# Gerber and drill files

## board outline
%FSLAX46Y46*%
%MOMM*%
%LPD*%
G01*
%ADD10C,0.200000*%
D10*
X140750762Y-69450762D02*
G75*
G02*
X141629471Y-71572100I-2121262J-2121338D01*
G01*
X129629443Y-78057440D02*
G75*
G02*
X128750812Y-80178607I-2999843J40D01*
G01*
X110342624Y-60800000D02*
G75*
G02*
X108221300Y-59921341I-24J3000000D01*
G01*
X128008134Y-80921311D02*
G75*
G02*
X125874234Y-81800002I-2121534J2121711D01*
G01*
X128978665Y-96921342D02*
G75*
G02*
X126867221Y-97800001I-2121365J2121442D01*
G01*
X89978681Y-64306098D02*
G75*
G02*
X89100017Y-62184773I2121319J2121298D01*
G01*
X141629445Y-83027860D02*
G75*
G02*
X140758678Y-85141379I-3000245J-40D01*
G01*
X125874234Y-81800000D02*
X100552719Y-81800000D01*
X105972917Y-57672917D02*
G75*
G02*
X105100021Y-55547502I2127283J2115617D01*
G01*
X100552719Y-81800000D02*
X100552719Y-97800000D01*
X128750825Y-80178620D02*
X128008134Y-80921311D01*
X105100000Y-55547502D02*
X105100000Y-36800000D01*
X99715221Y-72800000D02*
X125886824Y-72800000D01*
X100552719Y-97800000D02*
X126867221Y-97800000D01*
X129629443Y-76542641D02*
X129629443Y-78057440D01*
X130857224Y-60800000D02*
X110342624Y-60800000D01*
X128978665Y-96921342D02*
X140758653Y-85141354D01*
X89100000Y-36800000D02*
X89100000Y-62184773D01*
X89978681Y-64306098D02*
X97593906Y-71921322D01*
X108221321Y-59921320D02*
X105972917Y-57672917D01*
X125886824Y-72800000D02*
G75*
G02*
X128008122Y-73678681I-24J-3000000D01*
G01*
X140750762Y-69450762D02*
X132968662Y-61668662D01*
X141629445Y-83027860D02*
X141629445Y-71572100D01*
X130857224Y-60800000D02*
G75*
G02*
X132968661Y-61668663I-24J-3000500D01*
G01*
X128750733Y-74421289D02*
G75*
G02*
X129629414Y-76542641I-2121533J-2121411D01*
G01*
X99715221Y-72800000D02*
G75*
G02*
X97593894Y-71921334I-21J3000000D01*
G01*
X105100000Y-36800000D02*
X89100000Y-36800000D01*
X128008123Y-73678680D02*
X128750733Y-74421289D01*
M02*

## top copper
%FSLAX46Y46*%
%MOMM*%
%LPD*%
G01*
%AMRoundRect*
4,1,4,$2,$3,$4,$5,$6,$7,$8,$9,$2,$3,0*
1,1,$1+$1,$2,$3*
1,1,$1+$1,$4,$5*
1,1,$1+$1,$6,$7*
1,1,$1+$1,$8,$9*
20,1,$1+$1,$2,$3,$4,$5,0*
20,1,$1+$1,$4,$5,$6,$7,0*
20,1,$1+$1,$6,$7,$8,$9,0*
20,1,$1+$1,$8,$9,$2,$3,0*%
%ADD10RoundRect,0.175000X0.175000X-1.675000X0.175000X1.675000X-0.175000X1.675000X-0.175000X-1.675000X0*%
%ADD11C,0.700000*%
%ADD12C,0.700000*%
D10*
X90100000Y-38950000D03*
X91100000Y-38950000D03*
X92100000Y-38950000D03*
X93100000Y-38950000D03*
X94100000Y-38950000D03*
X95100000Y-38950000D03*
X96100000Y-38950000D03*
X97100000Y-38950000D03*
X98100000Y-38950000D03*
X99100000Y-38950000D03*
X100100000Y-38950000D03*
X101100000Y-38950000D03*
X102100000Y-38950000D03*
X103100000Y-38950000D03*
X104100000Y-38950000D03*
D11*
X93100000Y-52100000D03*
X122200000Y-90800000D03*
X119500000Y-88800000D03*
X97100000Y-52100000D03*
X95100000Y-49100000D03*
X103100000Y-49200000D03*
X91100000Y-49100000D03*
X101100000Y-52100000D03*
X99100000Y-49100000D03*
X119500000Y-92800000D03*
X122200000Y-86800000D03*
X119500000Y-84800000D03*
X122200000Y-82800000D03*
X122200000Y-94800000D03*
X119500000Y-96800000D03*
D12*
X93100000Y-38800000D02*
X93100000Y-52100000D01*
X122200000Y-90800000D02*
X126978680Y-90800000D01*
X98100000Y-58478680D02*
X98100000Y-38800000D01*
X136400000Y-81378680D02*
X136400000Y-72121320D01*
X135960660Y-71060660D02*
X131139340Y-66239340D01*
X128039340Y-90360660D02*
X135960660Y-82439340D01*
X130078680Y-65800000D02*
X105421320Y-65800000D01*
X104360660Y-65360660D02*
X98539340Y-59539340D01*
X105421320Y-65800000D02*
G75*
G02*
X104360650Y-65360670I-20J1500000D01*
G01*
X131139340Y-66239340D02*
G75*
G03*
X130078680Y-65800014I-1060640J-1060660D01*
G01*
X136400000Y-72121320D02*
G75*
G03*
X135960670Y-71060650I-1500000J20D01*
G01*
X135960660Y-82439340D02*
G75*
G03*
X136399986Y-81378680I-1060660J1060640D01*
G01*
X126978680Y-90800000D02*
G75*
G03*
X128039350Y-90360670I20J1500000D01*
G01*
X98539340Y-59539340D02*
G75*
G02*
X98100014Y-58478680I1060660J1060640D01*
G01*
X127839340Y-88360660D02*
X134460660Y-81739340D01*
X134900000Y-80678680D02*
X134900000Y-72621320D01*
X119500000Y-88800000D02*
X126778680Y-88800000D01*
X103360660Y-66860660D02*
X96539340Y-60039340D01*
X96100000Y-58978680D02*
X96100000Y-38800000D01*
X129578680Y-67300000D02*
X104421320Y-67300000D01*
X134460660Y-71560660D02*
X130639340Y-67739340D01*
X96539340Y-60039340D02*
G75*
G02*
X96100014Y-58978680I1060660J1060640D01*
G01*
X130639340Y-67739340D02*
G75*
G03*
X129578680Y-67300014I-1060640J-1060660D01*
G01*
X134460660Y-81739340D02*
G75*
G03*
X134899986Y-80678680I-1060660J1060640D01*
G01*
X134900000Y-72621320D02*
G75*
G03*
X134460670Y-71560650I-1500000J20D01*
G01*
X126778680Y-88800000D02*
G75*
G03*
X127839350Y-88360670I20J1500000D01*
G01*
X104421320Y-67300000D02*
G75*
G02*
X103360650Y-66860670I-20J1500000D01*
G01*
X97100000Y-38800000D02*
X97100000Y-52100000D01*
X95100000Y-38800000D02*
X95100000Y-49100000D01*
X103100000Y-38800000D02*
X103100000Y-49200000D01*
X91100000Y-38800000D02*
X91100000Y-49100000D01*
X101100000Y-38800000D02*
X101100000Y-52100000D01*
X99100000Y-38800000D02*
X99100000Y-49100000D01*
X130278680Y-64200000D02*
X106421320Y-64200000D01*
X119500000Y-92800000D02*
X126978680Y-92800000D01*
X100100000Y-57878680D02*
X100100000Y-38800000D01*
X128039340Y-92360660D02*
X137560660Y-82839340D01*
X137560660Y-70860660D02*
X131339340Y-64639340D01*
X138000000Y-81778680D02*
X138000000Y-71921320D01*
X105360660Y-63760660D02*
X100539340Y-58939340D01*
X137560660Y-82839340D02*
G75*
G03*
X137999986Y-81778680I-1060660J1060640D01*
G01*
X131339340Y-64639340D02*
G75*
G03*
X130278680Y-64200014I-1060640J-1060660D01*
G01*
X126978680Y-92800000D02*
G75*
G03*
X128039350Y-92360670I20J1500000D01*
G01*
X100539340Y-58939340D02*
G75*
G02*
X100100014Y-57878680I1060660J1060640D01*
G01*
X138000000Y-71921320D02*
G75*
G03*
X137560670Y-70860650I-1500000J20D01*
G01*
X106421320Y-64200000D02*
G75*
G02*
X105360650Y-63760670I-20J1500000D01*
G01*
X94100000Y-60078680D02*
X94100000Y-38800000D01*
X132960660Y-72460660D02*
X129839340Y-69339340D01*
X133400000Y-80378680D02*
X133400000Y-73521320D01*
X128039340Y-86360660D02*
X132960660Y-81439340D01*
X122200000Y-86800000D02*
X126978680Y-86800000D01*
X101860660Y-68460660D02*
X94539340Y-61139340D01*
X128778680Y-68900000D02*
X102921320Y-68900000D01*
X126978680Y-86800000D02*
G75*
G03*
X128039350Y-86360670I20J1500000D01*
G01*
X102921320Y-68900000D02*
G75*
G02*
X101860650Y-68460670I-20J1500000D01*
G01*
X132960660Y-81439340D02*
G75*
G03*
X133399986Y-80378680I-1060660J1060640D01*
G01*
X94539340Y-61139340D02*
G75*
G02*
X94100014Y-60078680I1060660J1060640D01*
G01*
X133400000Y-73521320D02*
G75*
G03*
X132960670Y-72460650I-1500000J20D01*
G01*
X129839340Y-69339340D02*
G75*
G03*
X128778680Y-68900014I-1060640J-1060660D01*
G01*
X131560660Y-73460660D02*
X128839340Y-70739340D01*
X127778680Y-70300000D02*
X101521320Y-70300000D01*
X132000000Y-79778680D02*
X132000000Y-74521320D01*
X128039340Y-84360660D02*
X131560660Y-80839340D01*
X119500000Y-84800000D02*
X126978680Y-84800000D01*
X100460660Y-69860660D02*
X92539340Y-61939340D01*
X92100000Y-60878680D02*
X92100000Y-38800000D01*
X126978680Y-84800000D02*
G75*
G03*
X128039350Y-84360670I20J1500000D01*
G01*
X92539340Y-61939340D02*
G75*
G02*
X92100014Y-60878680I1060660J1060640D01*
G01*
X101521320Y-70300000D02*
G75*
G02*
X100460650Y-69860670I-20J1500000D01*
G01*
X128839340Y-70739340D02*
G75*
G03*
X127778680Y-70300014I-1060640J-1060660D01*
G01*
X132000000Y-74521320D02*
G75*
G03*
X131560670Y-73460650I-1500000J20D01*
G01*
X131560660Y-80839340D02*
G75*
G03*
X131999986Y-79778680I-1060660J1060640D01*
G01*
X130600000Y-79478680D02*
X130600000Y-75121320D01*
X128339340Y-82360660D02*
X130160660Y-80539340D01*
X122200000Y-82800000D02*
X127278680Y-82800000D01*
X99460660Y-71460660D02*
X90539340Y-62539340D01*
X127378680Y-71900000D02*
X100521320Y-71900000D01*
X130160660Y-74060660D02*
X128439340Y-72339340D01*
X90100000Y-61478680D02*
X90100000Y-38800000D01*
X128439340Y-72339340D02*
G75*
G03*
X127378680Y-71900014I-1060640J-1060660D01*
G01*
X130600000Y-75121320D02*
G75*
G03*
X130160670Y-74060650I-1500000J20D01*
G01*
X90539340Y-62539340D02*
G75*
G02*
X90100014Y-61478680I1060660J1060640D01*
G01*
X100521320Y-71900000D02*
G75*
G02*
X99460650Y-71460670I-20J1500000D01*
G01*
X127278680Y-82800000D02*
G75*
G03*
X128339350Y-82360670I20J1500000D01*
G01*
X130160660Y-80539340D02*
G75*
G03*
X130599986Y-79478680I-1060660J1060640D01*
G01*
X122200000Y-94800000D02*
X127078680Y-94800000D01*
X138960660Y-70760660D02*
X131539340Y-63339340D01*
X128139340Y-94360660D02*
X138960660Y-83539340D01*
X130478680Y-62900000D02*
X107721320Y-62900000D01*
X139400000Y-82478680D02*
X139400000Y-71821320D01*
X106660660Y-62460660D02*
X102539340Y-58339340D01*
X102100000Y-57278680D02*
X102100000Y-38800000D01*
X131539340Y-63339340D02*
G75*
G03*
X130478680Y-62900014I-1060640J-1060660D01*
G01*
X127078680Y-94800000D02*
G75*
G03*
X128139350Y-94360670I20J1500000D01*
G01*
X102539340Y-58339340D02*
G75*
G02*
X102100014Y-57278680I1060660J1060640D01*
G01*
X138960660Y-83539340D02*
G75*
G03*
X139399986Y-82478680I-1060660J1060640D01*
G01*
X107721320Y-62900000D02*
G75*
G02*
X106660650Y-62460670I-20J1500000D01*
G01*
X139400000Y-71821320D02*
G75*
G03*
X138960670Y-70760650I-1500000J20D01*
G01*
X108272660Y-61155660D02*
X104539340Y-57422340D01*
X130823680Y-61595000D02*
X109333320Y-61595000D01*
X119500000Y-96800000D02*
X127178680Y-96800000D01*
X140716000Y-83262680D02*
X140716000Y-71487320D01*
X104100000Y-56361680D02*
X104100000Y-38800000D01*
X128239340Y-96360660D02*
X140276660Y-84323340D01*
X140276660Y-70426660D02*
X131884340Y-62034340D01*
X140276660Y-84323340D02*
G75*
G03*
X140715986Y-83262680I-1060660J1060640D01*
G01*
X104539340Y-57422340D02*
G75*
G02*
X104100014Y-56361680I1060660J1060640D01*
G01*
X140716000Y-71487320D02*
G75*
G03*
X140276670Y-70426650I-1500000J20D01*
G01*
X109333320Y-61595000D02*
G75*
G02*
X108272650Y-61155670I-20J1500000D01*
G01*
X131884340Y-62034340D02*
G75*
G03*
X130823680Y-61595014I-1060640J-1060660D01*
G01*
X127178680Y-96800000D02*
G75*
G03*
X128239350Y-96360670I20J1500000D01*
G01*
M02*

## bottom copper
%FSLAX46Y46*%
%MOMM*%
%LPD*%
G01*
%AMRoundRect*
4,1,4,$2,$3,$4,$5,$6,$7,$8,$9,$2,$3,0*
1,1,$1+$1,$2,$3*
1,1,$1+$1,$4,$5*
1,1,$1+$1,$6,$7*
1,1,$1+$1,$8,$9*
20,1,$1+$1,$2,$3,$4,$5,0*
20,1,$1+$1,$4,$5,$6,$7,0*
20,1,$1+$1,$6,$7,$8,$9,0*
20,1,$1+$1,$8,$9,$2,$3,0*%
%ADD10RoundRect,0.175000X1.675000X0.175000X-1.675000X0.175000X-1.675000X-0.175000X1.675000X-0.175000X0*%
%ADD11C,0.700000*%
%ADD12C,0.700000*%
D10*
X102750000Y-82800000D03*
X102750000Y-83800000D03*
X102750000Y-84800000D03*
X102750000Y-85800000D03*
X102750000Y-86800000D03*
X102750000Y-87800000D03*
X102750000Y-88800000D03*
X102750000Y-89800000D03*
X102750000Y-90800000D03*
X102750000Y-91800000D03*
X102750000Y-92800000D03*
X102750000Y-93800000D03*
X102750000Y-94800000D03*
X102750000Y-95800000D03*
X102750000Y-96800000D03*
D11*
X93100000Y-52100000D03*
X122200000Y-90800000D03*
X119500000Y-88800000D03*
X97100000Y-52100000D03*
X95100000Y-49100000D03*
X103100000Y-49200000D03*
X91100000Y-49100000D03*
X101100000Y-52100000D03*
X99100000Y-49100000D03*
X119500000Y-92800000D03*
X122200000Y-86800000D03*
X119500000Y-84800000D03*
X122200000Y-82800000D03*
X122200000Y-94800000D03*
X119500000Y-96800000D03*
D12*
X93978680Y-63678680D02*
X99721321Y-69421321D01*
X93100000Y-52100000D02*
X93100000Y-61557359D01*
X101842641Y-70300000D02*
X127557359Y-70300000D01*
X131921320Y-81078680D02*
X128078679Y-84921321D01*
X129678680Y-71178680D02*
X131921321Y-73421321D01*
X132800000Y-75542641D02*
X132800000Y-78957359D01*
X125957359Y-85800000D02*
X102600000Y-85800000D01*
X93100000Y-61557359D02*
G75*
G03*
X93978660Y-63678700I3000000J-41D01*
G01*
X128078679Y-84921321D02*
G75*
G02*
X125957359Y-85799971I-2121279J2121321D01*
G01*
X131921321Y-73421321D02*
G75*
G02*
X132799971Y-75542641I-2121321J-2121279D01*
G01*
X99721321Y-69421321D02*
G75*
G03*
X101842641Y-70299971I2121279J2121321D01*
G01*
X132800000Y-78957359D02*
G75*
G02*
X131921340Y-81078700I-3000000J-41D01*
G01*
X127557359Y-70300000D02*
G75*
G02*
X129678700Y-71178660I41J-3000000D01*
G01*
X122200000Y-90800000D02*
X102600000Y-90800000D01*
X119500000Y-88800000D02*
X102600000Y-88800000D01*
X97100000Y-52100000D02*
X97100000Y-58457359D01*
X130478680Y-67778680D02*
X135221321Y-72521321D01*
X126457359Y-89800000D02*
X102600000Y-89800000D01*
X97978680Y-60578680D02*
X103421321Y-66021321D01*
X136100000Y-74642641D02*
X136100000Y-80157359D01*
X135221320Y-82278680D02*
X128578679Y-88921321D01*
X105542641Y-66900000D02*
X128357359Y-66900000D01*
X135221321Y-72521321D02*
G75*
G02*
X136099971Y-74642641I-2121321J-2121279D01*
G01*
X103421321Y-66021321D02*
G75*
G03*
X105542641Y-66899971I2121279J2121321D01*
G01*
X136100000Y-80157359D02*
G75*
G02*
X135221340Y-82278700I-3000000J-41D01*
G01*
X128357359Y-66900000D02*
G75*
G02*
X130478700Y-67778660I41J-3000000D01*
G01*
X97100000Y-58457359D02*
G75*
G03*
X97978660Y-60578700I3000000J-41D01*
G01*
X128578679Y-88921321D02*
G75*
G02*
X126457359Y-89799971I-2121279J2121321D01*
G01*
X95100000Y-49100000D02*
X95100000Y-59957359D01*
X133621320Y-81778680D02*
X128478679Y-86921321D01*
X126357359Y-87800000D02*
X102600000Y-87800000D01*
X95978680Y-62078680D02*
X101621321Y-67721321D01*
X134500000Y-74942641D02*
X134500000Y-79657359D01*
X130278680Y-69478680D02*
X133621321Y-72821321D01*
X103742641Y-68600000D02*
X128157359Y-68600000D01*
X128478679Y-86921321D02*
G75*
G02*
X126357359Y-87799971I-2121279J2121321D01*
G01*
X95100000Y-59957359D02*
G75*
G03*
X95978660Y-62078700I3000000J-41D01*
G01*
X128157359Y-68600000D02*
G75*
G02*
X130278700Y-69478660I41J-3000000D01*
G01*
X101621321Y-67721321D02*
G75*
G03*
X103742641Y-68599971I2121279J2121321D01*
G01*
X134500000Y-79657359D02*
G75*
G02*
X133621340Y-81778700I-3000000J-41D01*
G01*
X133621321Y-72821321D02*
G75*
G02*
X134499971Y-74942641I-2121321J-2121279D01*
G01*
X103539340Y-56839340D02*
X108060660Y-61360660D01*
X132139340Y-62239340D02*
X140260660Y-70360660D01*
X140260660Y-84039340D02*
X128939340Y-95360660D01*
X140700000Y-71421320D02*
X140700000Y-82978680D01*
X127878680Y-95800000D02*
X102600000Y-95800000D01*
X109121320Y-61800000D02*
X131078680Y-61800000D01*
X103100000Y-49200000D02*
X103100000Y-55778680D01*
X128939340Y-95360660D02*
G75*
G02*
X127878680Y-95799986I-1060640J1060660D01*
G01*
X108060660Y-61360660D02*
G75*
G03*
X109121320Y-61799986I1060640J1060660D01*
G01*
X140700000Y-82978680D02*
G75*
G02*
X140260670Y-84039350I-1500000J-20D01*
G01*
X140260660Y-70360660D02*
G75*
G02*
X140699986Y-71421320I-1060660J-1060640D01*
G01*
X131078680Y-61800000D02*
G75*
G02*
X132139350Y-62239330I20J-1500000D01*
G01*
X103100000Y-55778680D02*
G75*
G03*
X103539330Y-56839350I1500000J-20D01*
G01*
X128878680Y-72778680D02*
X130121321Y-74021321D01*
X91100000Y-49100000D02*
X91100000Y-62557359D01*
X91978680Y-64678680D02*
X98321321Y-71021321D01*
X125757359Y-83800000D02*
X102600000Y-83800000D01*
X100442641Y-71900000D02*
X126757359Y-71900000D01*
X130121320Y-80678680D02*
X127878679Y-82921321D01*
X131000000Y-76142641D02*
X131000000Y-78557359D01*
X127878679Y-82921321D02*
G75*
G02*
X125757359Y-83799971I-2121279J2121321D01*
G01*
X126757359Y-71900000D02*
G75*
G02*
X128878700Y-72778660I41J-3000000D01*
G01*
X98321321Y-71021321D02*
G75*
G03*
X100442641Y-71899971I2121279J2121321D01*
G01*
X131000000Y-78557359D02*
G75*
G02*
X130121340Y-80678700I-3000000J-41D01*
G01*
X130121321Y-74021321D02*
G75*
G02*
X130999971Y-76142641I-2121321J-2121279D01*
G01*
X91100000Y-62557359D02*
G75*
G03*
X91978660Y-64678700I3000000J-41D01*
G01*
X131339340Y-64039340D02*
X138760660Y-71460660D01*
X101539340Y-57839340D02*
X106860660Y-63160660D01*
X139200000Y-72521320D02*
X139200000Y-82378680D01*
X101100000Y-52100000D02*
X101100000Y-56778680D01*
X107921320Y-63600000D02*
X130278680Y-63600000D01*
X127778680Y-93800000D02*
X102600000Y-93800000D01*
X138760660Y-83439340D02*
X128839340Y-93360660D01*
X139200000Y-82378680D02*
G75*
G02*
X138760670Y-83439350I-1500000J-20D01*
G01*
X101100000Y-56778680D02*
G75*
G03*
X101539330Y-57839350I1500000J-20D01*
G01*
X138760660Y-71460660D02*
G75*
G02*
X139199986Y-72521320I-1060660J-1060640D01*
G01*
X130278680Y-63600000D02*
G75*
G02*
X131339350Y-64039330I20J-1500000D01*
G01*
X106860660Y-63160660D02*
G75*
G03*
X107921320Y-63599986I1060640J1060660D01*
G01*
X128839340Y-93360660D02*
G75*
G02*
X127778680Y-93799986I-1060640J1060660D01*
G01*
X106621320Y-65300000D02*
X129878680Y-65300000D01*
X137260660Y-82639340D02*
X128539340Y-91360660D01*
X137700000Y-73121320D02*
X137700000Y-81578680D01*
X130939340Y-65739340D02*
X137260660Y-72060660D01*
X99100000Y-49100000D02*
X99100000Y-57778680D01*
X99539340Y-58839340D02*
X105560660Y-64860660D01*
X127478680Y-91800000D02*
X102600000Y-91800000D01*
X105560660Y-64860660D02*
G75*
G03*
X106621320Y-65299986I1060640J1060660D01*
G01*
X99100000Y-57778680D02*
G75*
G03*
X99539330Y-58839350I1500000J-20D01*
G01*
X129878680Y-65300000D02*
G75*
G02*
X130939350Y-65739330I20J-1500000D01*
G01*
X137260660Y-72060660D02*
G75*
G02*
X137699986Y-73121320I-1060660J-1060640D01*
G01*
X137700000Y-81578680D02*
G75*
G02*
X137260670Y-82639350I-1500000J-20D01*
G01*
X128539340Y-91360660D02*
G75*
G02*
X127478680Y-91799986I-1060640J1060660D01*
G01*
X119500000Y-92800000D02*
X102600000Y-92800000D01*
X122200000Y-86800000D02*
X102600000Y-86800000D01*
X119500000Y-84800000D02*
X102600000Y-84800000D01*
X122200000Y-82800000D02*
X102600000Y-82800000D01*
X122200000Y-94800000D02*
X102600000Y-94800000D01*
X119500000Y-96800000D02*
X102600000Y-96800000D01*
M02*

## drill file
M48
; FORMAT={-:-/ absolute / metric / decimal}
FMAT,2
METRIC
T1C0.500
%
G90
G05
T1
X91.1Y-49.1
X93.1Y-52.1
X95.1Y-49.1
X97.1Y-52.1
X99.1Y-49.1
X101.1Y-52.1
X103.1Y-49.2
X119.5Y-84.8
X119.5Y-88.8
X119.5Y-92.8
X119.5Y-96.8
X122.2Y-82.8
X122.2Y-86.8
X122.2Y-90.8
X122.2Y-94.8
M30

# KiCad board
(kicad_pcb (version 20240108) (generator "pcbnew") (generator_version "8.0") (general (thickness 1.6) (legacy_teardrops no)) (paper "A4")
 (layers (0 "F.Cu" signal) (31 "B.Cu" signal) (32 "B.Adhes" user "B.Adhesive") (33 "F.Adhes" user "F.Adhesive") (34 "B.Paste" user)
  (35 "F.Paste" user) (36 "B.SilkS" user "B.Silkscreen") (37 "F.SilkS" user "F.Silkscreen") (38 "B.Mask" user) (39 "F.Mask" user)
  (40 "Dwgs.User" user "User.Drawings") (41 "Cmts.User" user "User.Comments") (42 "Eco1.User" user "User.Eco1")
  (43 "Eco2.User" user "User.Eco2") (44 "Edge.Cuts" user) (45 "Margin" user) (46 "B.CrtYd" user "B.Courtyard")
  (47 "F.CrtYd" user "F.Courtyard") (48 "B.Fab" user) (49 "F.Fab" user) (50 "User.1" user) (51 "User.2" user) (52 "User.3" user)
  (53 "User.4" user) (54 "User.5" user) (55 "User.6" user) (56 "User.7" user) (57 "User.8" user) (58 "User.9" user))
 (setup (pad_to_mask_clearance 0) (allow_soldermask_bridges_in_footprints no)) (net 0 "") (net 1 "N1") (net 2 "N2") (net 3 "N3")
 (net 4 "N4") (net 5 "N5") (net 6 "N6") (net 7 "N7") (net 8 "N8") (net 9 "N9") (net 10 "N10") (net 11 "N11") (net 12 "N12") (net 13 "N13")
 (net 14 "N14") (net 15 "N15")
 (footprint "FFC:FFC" (layer "F.Cu") (at 97.1 38.8 90)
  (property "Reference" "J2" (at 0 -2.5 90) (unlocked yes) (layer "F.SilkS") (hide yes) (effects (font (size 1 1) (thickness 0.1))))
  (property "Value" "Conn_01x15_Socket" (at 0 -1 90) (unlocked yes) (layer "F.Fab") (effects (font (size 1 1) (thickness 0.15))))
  (pad "1" smd roundrect (at -0.15 -7 90) (size 3.7 0.7) (layers "F.Cu" "F.Paste" "F.Mask") (roundrect_rratio 0.25) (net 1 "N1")
   (thermal_bridge_angle 45))
  (pad "2" smd roundrect (at -0.15 -6 90) (size 3.7 0.7) (layers "F.Cu" "F.Paste" "F.Mask") (roundrect_rratio 0.25) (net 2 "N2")
   (thermal_bridge_angle 45))
  (pad "3" smd roundrect (at -0.15 -5 90) (size 3.7 0.7) (layers "F.Cu" "F.Paste" "F.Mask") (roundrect_rratio 0.25) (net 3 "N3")
   (thermal_bridge_angle 45))
  (pad "4" smd roundrect (at -0.15 -4 90) (size 3.7 0.7) (layers "F.Cu" "F.Paste" "F.Mask") (roundrect_rratio 0.25) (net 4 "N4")
   (thermal_bridge_angle 45))
  (pad "5" smd roundrect (at -0.15 -3 90) (size 3.7 0.7) (layers "F.Cu" "F.Paste" "F.Mask") (roundrect_rratio 0.25) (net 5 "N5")
   (thermal_bridge_angle 45))
  (pad "6" smd roundrect (at -0.15 -2 90) (size 3.7 0.7) (layers "F.Cu" "F.Paste" "F.Mask") (roundrect_rratio 0.25) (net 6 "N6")
   (thermal_bridge_angle 45))
  (pad "7" smd roundrect (at -0.15 -1 90) (size 3.7 0.7) (layers "F.Cu" "F.Paste" "F.Mask") (roundrect_rratio 0.25) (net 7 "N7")
   (thermal_bridge_angle 45))
  (pad "8" smd roundrect (at -0.15 0 90) (size 3.7 0.7) (layers "F.Cu" "F.Paste" "F.Mask") (roundrect_rratio 0.25) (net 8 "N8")
   (thermal_bridge_angle 45))
  (pad "9" smd roundrect (at -0.15 1 90) (size 3.7 0.7) (layers "F.Cu" "F.Paste" "F.Mask") (roundrect_rratio 0.25) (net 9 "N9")
   (thermal_bridge_angle 45))
  (pad "10" smd roundrect (at -0.15 2 90) (size 3.7 0.7) (layers "F.Cu" "F.Paste" "F.Mask") (roundrect_rratio 0.25) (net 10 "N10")
   (thermal_bridge_angle 45))
  (pad "11" smd roundrect (at -0.15 3 90) (size 3.7 0.7) (layers "F.Cu" "F.Paste" "F.Mask") (roundrect_rratio 0.25) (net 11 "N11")
   (thermal_bridge_angle 45))
  (pad "12" smd roundrect (at -0.15 4 90) (size 3.7 0.7) (layers "F.Cu" "F.Paste" "F.Mask") (roundrect_rratio 0.25) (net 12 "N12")
   (thermal_bridge_angle 45))
  (pad "13" smd roundrect (at -0.15 5 90) (size 3.7 0.7) (layers "F.Cu" "F.Paste" "F.Mask") (roundrect_rratio 0.25) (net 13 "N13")
   (thermal_bridge_angle 45))
  (pad "14" smd roundrect (at -0.15 6 90) (size 3.7 0.7) (layers "F.Cu" "F.Paste" "F.Mask") (roundrect_rratio 0.25) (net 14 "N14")
   (thermal_bridge_angle 45))
  (pad "15" smd roundrect (at -0.15 7 90) (size 3.7 0.7) (layers "F.Cu" "F.Paste" "F.Mask") (roundrect_rratio 0.25) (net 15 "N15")
   (thermal_bridge_angle 45)))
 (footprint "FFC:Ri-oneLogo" (layer "F.Cu") (at 111.1 69.2)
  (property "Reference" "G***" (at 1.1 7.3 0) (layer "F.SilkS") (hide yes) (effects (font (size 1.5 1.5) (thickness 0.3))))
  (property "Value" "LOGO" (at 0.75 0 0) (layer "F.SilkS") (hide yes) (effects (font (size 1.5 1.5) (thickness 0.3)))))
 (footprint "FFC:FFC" (layer "B.Cu") (at 102.6 89.8 180)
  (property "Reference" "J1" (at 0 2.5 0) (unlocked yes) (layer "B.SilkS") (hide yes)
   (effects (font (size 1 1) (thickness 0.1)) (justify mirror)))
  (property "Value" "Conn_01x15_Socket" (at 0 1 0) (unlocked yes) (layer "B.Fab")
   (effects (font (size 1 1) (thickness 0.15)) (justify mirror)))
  (pad "1" smd roundrect (at -0.15 7 180) (size 3.7 0.7) (layers "B.Cu" "B.Paste" "B.Mask") (roundrect_rratio 0.25) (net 1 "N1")
   (thermal_bridge_angle 45))
  (pad "2" smd roundrect (at -0.15 6 180) (size 3.7 0.7) (layers "B.Cu" "B.Paste" "B.Mask") (roundrect_rratio 0.25) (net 2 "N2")
   (thermal_bridge_angle 45))
  (pad "3" smd roundrect (at -0.15 5 180) (size 3.7 0.7) (layers "B.Cu" "B.Paste" "B.Mask") (roundrect_rratio 0.25) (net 3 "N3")
   (thermal_bridge_angle 45))
  (pad "4" smd roundrect (at -0.15 4 180) (size 3.7 0.7) (layers "B.Cu" "B.Paste" "B.Mask") (roundrect_rratio 0.25) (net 4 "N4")
   (thermal_bridge_angle 45))
  (pad "5" smd roundrect (at -0.15 3 180) (size 3.7 0.7) (layers "B.Cu" "B.Paste" "B.Mask") (roundrect_rratio 0.25) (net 5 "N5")
   (thermal_bridge_angle 45))
  (pad "6" smd roundrect (at -0.15 2 180) (size 3.7 0.7) (layers "B.Cu" "B.Paste" "B.Mask") (roundrect_rratio 0.25) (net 6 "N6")
   (thermal_bridge_angle 45))
  (pad "7" smd roundrect (at -0.15 1 180) (size 3.7 0.7) (layers "B.Cu" "B.Paste" "B.Mask") (roundrect_rratio 0.25) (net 7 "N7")
   (thermal_bridge_angle 45))
  (pad "8" smd roundrect (at -0.15 0 180) (size 3.7 0.7) (layers "B.Cu" "B.Paste" "B.Mask") (roundrect_rratio 0.25) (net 8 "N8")
   (thermal_bridge_angle 45))
  (pad "9" smd roundrect (at -0.15 -1 180) (size 3.7 0.7) (layers "B.Cu" "B.Paste" "B.Mask") (roundrect_rratio 0.25) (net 9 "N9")
   (thermal_bridge_angle 45))
  (pad "10" smd roundrect (at -0.15 -2 180) (size 3.7 0.7) (layers "B.Cu" "B.Paste" "B.Mask") (roundrect_rratio 0.25) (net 10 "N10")
   (thermal_bridge_angle 45))
  (pad "11" smd roundrect (at -0.15 -3 180) (size 3.7 0.7) (layers "B.Cu" "B.Paste" "B.Mask") (roundrect_rratio 0.25) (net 11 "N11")
   (thermal_bridge_angle 45))
  (pad "12" smd roundrect (at -0.15 -4 180) (size 3.7 0.7) (layers "B.Cu" "B.Paste" "B.Mask") (roundrect_rratio 0.25) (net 12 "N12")
   (thermal_bridge_angle 45))
  (pad "13" smd roundrect (at -0.15 -5 180) (size 3.7 0.7) (layers "B.Cu" "B.Paste" "B.Mask") (roundrect_rratio 0.25) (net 13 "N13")
   (thermal_bridge_angle 45))
  (pad "14" smd roundrect (at -0.15 -6 180) (size 3.7 0.7) (layers "B.Cu" "B.Paste" "B.Mask") (roundrect_rratio 0.25) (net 14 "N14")
   (thermal_bridge_angle 45))
  (pad "15" smd roundrect (at -0.15 -7 180) (size 3.7 0.7) (layers "B.Cu" "B.Paste" "B.Mask") (roundrect_rratio 0.25) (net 15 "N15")
   (thermal_bridge_angle 45)))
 (gr_arc (start 140.750762 69.450762) (mid 141.401086 70.42404) (end 141.629445 71.5721) (stroke (width 0.2) (type default))
  (layer "Edge.Cuts"))
 (gr_arc (start 129.629443 78.05744) (mid 129.401097 79.205413) (end 128.750825 80.17862) (stroke (width 0.2) (type default))
  (layer "Edge.Cuts"))
 (gr_arc (start 110.342624 60.8) (mid 109.194585 60.571635) (end 108.221321 59.92132) (stroke (width 0.2) (type default))
  (layer "Edge.Cuts"))
 (gr_arc (start 128.008134 80.921311) (mid 127.029045 81.574019) (end 125.874234 81.8) (stroke (width 0.2) (type default))
  (layer "Edge.Cuts"))
 (gr_arc (start 128.978665 96.921342) (mid 128.009955 97.569757) (end 126.867221 97.8) (stroke (width 0.2) (type default))
  (layer "Edge.Cuts"))
 (gr_arc (start 89.978681 64.306098) (mid 89.328361 63.332826) (end 89.1 62.184773) (stroke (width 0.2) (type default)) (layer "Edge.Cuts"))
 (gr_arc (start 141.629445 83.02786) (mid 141.403217 84.170787) (end 140.758653 85.141354) (stroke (width 0.2) (type default))
  (layer "Edge.Cuts"))
 (gr_line (start 125.874234 81.8) (end 100.552719 81.8) (stroke (width 0.2) (type default)) (layer "Edge.Cuts"))
 (gr_arc (start 105.972917 57.672917) (mid 105.324931 56.697085) (end 105.1 55.547502) (stroke (width 0.2) (type default))
  (layer "Edge.Cuts"))
 (gr_line (start 100.552719 81.8) (end 100.552719 97.8) (stroke (width 0.2) (type default)) (layer "Edge.Cuts"))
 (gr_line (start 128.750825 80.17862) (end 128.008134 80.921311) (stroke (width 0.2) (type default)) (layer "Edge.Cuts"))
 (gr_line (start 105.1 55.547502) (end 105.1 36.8) (stroke (width 0.2) (type default)) (layer "Edge.Cuts"))
 (gr_line (start 99.715221 72.8) (end 125.886824 72.8) (stroke (width 0.2) (type default)) (layer "Edge.Cuts"))
 (gr_line (start 100.552719 97.8) (end 126.867221 97.8) (stroke (width 0.2) (type default)) (layer "Edge.Cuts"))
 (gr_line (start 129.629443 76.542641) (end 129.629443 78.05744) (stroke (width 0.2) (type default)) (layer "Edge.Cuts"))
 (gr_line (start 130.857224 60.8) (end 110.342624 60.8) (stroke (width 0.2) (type default)) (layer "Edge.Cuts"))
 (gr_line (start 128.978665 96.921342) (end 140.758653 85.141354) (stroke (width 0.2) (type default)) (layer "Edge.Cuts"))
 (gr_line (start 89.1 36.8) (end 89.1 62.184773) (stroke (width 0.2) (type default)) (layer "Edge.Cuts"))
 (gr_line (start 89.978681 64.306098) (end 97.593906 71.921322) (stroke (width 0.2) (type default)) (layer "Edge.Cuts"))
 (gr_line (start 108.221321 59.92132) (end 105.972917 57.672917) (stroke (width 0.2) (type default)) (layer "Edge.Cuts"))
 (gr_arc (start 125.886824 72.8) (mid 127.034862 73.028364) (end 128.008123 73.67868) (stroke (width 0.2) (type default))
  (layer "Edge.Cuts"))
 (gr_line (start 140.750762 69.450762) (end 132.968662 61.668662) (stroke (width 0.2) (type default)) (layer "Edge.Cuts"))
 (gr_line (start 141.629445 83.02786) (end 141.629445 71.5721) (stroke (width 0.2) (type default)) (layer "Edge.Cuts"))
 (gr_arc (start 130.857224 60.8) (mid 131.998793 61.025653) (end 132.968662 61.668662) (stroke (width 0.2) (type default))
  (layer "Edge.Cuts"))
 (gr_arc (start 128.750733 74.421289) (mid 129.401057 75.394574) (end 129.629443 76.542641) (stroke (width 0.2) (type default))
  (layer "Edge.Cuts"))
 (gr_arc (start 99.715221 72.8) (mid 98.567174 72.571639) (end 97.593906 71.921322) (stroke (width 0.2) (type default)) (layer "Edge.Cuts"))
 (gr_line (start 105.1 36.8) (end 89.1 36.8) (stroke (width 0.2) (type default)) (layer "Edge.Cuts"))
 (gr_line (start 128.008123 73.67868) (end 128.750733 74.421289) (stroke (width 0.2) (type default)) (layer "Edge.Cuts"))
 (segment (start 93.1 38.8) (end 93.1 52.1) (width 0.7) (layer "F.Cu") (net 4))
 (via (at 93.1 52.1) (size 0.7) (drill 0.5) (layers "F.Cu" "B.Cu") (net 4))
 (segment (start 93.97868 63.67868) (end 99.721321 69.421321) (width 0.7) (layer "B.Cu") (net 4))
 (segment (start 93.1 52.1) (end 93.1 61.557359) (width 0.7) (layer "B.Cu") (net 4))
 (segment (start 101.842641 70.3) (end 127.557359 70.3) (width 0.7) (layer "B.Cu") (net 4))
 (segment (start 131.92132 81.07868) (end 128.078679 84.921321) (width 0.7) (layer "B.Cu") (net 4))
 (segment (start 129.67868 71.17868) (end 131.921321 73.421321) (width 0.7) (layer "B.Cu") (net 4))
 (segment (start 132.8 75.542641) (end 132.8 78.957359) (width 0.7) (layer "B.Cu") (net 4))
 (segment (start 125.957359 85.8) (end 102.6 85.8) (width 0.7) (layer "B.Cu") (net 4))
 (arc (start 93.1 61.557359) (mid 93.328362 62.70541) (end 93.97868 63.67868) (width 0.7) (layer "B.Cu") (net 4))
 (arc (start 128.078679 84.921321) (mid 127.105409 85.571639) (end 125.957359 85.8) (width 0.7) (layer "B.Cu") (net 4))
 (arc (start 131.921321 73.421321) (mid 132.571639 74.394591) (end 132.8 75.542641) (width 0.7) (layer "B.Cu") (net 4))
 (arc (start 99.721321 69.421321) (mid 100.694591 70.071639) (end 101.842641 70.3) (width 0.7) (layer "B.Cu") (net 4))
 (arc (start 132.8 78.957359) (mid 132.571638 80.10541) (end 131.92132 81.07868) (width 0.7) (layer "B.Cu") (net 4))
 (arc (start 127.557359 70.3) (mid 128.70541 70.528362) (end 129.67868 71.17868) (width 0.7) (layer "B.Cu") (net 4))
 (segment (start 122.2 90.8) (end 126.97868 90.8) (width 0.7) (layer "F.Cu") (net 9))
 (segment (start 98.1 58.47868) (end 98.1 38.8) (width 0.7) (layer "F.Cu") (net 9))
 (segment (start 136.4 81.37868) (end 136.4 72.12132) (width 0.7) (layer "F.Cu") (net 9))
 (segment (start 135.96066 71.06066) (end 131.13934 66.23934) (width 0.7) (layer "F.Cu") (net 9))
 (segment (start 128.03934 90.36066) (end 135.96066 82.43934) (width 0.7) (layer "F.Cu") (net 9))
 (segment (start 130.07868 65.8) (end 105.42132 65.8) (width 0.7) (layer "F.Cu") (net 9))
 (segment (start 104.36066 65.36066) (end 98.53934 59.53934) (width 0.7) (layer "F.Cu") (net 9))
 (via (at 122.2 90.8) (size 0.7) (drill 0.5) (layers "F.Cu" "B.Cu") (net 9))
 (arc (start 105.42132 65.8) (mid 104.847295 65.685819) (end 104.36066 65.36066) (width 0.7) (layer "F.Cu") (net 9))
 (arc (start 131.13934 66.23934) (mid 130.652705 65.914181) (end 130.07868 65.8) (width 0.7) (layer "F.Cu") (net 9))
 (arc (start 136.4 72.12132) (mid 136.285819 71.547295) (end 135.96066 71.06066) (width 0.7) (layer "F.Cu") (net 9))
 (arc (start 135.96066 82.43934) (mid 136.285819 81.952705) (end 136.4 81.37868) (width 0.7) (layer "F.Cu") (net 9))
 (arc (start 126.97868 90.8) (mid 127.552705 90.685819) (end 128.03934 90.36066) (width 0.7) (layer "F.Cu") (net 9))
 (arc (start 98.53934 59.53934) (mid 98.214181 59.052705) (end 98.1 58.47868) (width 0.7) (layer "F.Cu") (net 9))
 (segment (start 122.2 90.8) (end 102.6 90.8) (width 0.7) (layer "B.Cu") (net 9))
 (segment (start 127.83934 88.36066) (end 134.46066 81.73934) (width 0.7) (layer "F.Cu") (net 7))
 (segment (start 134.9 80.67868) (end 134.9 72.62132) (width 0.7) (layer "F.Cu") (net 7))
 (segment (start 119.5 88.8) (end 126.77868 88.8) (width 0.7) (layer "F.Cu") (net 7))
 (segment (start 103.36066 66.86066) (end 96.53934 60.03934) (width 0.7) (layer "F.Cu") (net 7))
 (segment (start 96.1 58.97868) (end 96.1 38.8) (width 0.7) (layer "F.Cu") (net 7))
 (segment (start 129.57868 67.3) (end 104.42132 67.3) (width 0.7) (layer "F.Cu") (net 7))
 (segment (start 134.46066 71.56066) (end 130.63934 67.73934) (width 0.7) (layer "F.Cu") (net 7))
 (via (at 119.5 88.8) (size 0.7) (drill 0.5) (layers "F.Cu" "B.Cu") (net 7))
 (arc (start 96.53934 60.03934) (mid 96.214181 59.552705) (end 96.1 58.97868) (width 0.7) (layer "F.Cu") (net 7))
 (arc (start 130.63934 67.73934) (mid 130.152705 67.414181) (end 129.57868 67.3) (width 0.7) (layer "F.Cu") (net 7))
 (arc (start 134.46066 81.73934) (mid 134.785819 81.252705) (end 134.9 80.67868) (width 0.7) (layer "F.Cu") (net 7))
 (arc (start 134.9 72.62132) (mid 134.785819 72.047295) (end 134.46066 71.56066) (width 0.7) (layer "F.Cu") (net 7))
 (arc (start 126.77868 88.8) (mid 127.352705 88.685819) (end 127.83934 88.36066) (width 0.7) (layer "F.Cu") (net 7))
 (arc (start 104.42132 67.3) (mid 103.847295 67.185819) (end 103.36066 66.86066) (width 0.7) (layer "F.Cu") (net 7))
 (segment (start 119.5 88.8) (end 102.6 88.8) (width 0.7) (layer "B.Cu") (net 7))
 (segment (start 97.1 38.8) (end 97.1 52.1) (width 0.7) (layer "F.Cu") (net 8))
 (via (at 97.1 52.1) (size 0.7) (drill 0.5) (layers "F.Cu" "B.Cu") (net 8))
 (segment (start 97.1 52.1) (end 97.1 58.457359) (width 0.7) (layer "B.Cu") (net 8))
 (segment (start 130.47868 67.77868) (end 135.221321 72.521321) (width 0.7) (layer "B.Cu") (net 8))
 (segment (start 126.457359 89.8) (end 102.6 89.8) (width 0.7) (layer "B.Cu") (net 8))
 (segment (start 97.97868 60.57868) (end 103.421321 66.021321) (width 0.7) (layer "B.Cu") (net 8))
 (segment (start 136.1 74.642641) (end 136.1 80.157359) (width 0.7) (layer "B.Cu") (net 8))
 (segment (start 135.22132 82.27868) (end 128.578679 88.921321) (width 0.7) (layer "B.Cu") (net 8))
 (segment (start 105.542641 66.9) (end 128.357359 66.9) (width 0.7) (layer "B.Cu") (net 8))
 (arc (start 135.221321 72.521321) (mid 135.871639 73.494591) (end 136.1 74.642641) (width 0.7) (layer "B.Cu") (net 8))
 (arc (start 103.421321 66.021321) (mid 104.394591 66.671639) (end 105.542641 66.9) (width 0.7) (layer "B.Cu") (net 8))
 (arc (start 136.1 80.157359) (mid 135.871639 81.30541) (end 135.22132 82.27868) (width 0.7) (layer "B.Cu") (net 8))
 (arc (start 128.357359 66.9) (mid 129.50541 67.128362) (end 130.47868 67.77868) (width 0.7) (layer "B.Cu") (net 8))
 (arc (start 97.1 58.457359) (mid 97.328362 59.60541) (end 97.97868 60.57868) (width 0.7) (layer "B.Cu") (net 8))
 (arc (start 128.578679 88.921321) (mid 127.605409 89.571639) (end 126.457359 89.8) (width 0.7) (layer "B.Cu") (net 8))
 (segment (start 95.1 38.8) (end 95.1 49.1) (width 0.7) (layer "F.Cu") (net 6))
 (via (at 95.1 49.1) (size 0.7) (drill 0.5) (layers "F.Cu" "B.Cu") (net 6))
 (segment (start 95.1 49.1) (end 95.1 59.957359) (width 0.7) (layer "B.Cu") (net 6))
 (segment (start 133.62132 81.77868) (end 128.478679 86.921321) (width 0.7) (layer "B.Cu") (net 6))
 (segment (start 126.357359 87.8) (end 102.6 87.8) (width 0.7) (layer "B.Cu") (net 6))
 (segment (start 95.97868 62.07868) (end 101.621321 67.721321) (width 0.7) (layer "B.Cu") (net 6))
 (segment (start 134.5 74.942641) (end 134.5 79.657359) (width 0.7) (layer "B.Cu") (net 6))
 (segment (start 130.27868 69.47868) (end 133.621321 72.821321) (width 0.7) (layer "B.Cu") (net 6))
 (segment (start 103.742641 68.6) (end 128.157359 68.6) (width 0.7) (layer "B.Cu") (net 6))
 (arc (start 128.478679 86.921321) (mid 127.505409 87.571639) (end 126.357359 87.8) (width 0.7) (layer "B.Cu") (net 6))
 (arc (start 95.1 59.957359) (mid 95.328361 61.10541) (end 95.97868 62.07868) (width 0.7) (layer "B.Cu") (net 6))
 (arc (start 128.157359 68.6) (mid 129.30541 68.828361) (end 130.27868 69.47868) (width 0.7) (layer "B.Cu") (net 6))
 (arc (start 101.621321 67.721321) (mid 102.594591 68.371639) (end 103.742641 68.6) (width 0.7) (layer "B.Cu") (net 6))
 (arc (start 134.5 79.657359) (mid 134.271639 80.80541) (end 133.62132 81.77868) (width 0.7) (layer "B.Cu") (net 6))
 (arc (start 133.621321 72.821321) (mid 134.271639 73.794591) (end 134.5 74.942641) (width 0.7) (layer "B.Cu") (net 6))
 (segment (start 103.1 38.8) (end 103.1 49.2) (width 0.7) (layer "F.Cu") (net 14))
 (via (at 103.1 49.2) (size 0.7) (drill 0.5) (layers "F.Cu" "B.Cu") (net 14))
 (segment (start 103.53934 56.83934) (end 108.06066 61.36066) (width 0.7) (layer "B.Cu") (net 14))
 (segment (start 132.13934 62.23934) (end 140.26066 70.36066) (width 0.7) (layer "B.Cu") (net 14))
 (segment (start 140.26066 84.03934) (end 128.93934 95.36066) (width 0.7) (layer "B.Cu") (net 14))
 (segment (start 140.7 71.42132) (end 140.7 82.97868) (width 0.7) (layer "B.Cu") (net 14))
 (segment (start 127.87868 95.8) (end 102.6 95.8) (width 0.7) (layer "B.Cu") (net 14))
 (segment (start 109.12132 61.8) (end 131.07868 61.8) (width 0.7) (layer "B.Cu") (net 14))
 (segment (start 103.1 49.2) (end 103.1 55.77868) (width 0.7) (layer "B.Cu") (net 14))
 (arc (start 128.93934 95.36066) (mid 128.452705 95.685819) (end 127.87868 95.8) (width 0.7) (layer "B.Cu") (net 14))
 (arc (start 108.06066 61.36066) (mid 108.547295 61.685819) (end 109.12132 61.8) (width 0.7) (layer "B.Cu") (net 14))
 (arc (start 140.7 82.97868) (mid 140.585819 83.552705) (end 140.26066 84.03934) (width 0.7) (layer "B.Cu") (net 14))
 (arc (start 140.26066 70.36066) (mid 140.585819 70.847295) (end 140.7 71.42132) (width 0.7) (layer "B.Cu") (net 14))
 (arc (start 131.07868 61.8) (mid 131.652705 61.914181) (end 132.13934 62.23934) (width 0.7) (layer "B.Cu") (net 14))
 (arc (start 103.1 55.77868) (mid 103.214181 56.352705) (end 103.53934 56.83934) (width 0.7) (layer "B.Cu") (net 14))
 (segment (start 91.1 38.8) (end 91.1 49.1) (width 0.7) (layer "F.Cu") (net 2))
 (via (at 91.1 49.1) (size 0.7) (drill 0.5) (layers "F.Cu" "B.Cu") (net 2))
 (segment (start 128.87868 72.77868) (end 130.121321 74.021321) (width 0.7) (layer "B.Cu") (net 2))
 (segment (start 91.1 49.1) (end 91.1 62.557359) (width 0.7) (layer "B.Cu") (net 2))
 (segment (start 91.97868 64.67868) (end 98.321321 71.021321) (width 0.7) (layer "B.Cu") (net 2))
 (segment (start 125.757359 83.8) (end 102.6 83.8) (width 0.7) (layer "B.Cu") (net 2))
 (segment (start 100.442641 71.9) (end 126.757359 71.9) (width 0.7) (layer "B.Cu") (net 2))
 (segment (start 130.12132 80.67868) (end 127.878679 82.921321) (width 0.7) (layer "B.Cu") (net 2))
 (segment (start 131 76.142641) (end 131 78.557359) (width 0.7) (layer "B.Cu") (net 2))
 (arc (start 127.878679 82.921321) (mid 126.905409 83.571639) (end 125.757359 83.8) (width 0.7) (layer "B.Cu") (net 2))
 (arc (start 126.757359 71.9) (mid 127.90541 72.128361) (end 128.87868 72.77868) (width 0.7) (layer "B.Cu") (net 2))
 (arc (start 98.321321 71.021321) (mid 99.294591 71.671639) (end 100.442641 71.9) (width 0.7) (layer "B.Cu") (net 2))
 (arc (start 131 78.557359) (mid 130.771639 79.70541) (end 130.12132 80.67868) (width 0.7) (layer "B.Cu") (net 2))
 (arc (start 130.121321 74.021321) (mid 130.771639 74.994591) (end 131 76.142641) (width 0.7) (layer "B.Cu") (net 2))
 (arc (start 91.1 62.557359) (mid 91.328362 63.70541) (end 91.97868 64.67868) (width 0.7) (layer "B.Cu") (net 2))
 (segment (start 101.1 38.8) (end 101.1 52.1) (width 0.7) (layer "F.Cu") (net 12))
 (via (at 101.1 52.1) (size 0.7) (drill 0.5) (layers "F.Cu" "B.Cu") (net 12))
 (segment (start 131.33934 64.03934) (end 138.76066 71.46066) (width 0.7) (layer "B.Cu") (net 12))
 (segment (start 101.53934 57.83934) (end 106.86066 63.16066) (width 0.7) (layer "B.Cu") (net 12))
 (segment (start 139.2 72.52132) (end 139.2 82.37868) (width 0.7) (layer "B.Cu") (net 12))
 (segment (start 101.1 52.1) (end 101.1 56.77868) (width 0.7) (layer "B.Cu") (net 12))
 (segment (start 107.92132 63.6) (end 130.27868 63.6) (width 0.7) (layer "B.Cu") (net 12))
 (segment (start 127.77868 93.8) (end 102.6 93.8) (width 0.7) (layer "B.Cu") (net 12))
 (segment (start 138.76066 83.43934) (end 128.83934 93.36066) (width 0.7) (layer "B.Cu") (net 12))
 (arc (start 139.2 82.37868) (mid 139.085819 82.952705) (end 138.76066 83.43934) (width 0.7) (layer "B.Cu") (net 12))
 (arc (start 101.1 56.77868) (mid 101.214181 57.352705) (end 101.53934 57.83934) (width 0.7) (layer "B.Cu") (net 12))
 (arc (start 138.76066 71.46066) (mid 139.085819 71.947295) (end 139.2 72.52132) (width 0.7) (layer "B.Cu") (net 12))
 (arc (start 130.27868 63.6) (mid 130.852705 63.714181) (end 131.33934 64.03934) (width 0.7) (layer "B.Cu") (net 12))
 (arc (start 106.86066 63.16066) (mid 107.347295 63.485819) (end 107.92132 63.6) (width 0.7) (layer "B.Cu") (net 12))
 (arc (start 128.83934 93.36066) (mid 128.352705 93.685819) (end 127.77868 93.8) (width 0.7) (layer "B.Cu") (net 12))
 (segment (start 99.1 38.8) (end 99.1 49.1) (width 0.7) (layer "F.Cu") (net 10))
 (via (at 99.1 49.1) (size 0.7) (drill 0.5) (layers "F.Cu" "B.Cu") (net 10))
 (segment (start 106.62132 65.3) (end 129.87868 65.3) (width 0.7) (layer "B.Cu") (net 10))
 (segment (start 137.26066 82.63934) (end 128.53934 91.36066) (width 0.7) (layer "B.Cu") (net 10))
 (segment (start 137.7 73.12132) (end 137.7 81.57868) (width 0.7) (layer "B.Cu") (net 10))
 (segment (start 130.93934 65.73934) (end 137.26066 72.06066) (width 0.7) (layer "B.Cu") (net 10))
 (segment (start 99.1 49.1) (end 99.1 57.77868) (width 0.7) (layer "B.Cu") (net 10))
 (segment (start 99.53934 58.83934) (end 105.56066 64.86066) (width 0.7) (layer "B.Cu") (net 10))
 (segment (start 127.47868 91.8) (end 102.6 91.8) (width 0.7) (layer "B.Cu") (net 10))
 (arc (start 105.56066 64.86066) (mid 106.047295 65.185819) (end 106.62132 65.3) (width 0.7) (layer "B.Cu") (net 10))
 (arc (start 99.1 57.77868) (mid 99.214181 58.352705) (end 99.53934 58.83934) (width 0.7) (layer "B.Cu") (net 10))
 (arc (start 129.87868 65.3) (mid 130.452705 65.414181) (end 130.93934 65.73934) (width 0.7) (layer "B.Cu") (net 10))
 (arc (start 137.26066 72.06066) (mid 137.585819 72.547295) (end 137.7 73.12132) (width 0.7) (layer "B.Cu") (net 10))
 (arc (start 137.7 81.57868) (mid 137.585819 82.152705) (end 137.26066 82.63934) (width 0.7) (layer "B.Cu") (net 10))
 (arc (start 128.53934 91.36066) (mid 128.052705 91.685819) (end 127.47868 91.8) (width 0.7) (layer "B.Cu") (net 10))
 (segment (start 130.27868 64.2) (end 106.42132 64.2) (width 0.7) (layer "F.Cu") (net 11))
 (segment (start 119.5 92.8) (end 126.97868 92.8) (width 0.7) (layer "F.Cu") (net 11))
 (segment (start 100.1 57.87868) (end 100.1 38.8) (width 0.7) (layer "F.Cu") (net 11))
 (segment (start 128.03934 92.36066) (end 137.56066 82.83934) (width 0.7) (layer "F.Cu") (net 11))
 (segment (start 137.56066 70.86066) (end 131.33934 64.63934) (width 0.7) (layer "F.Cu") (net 11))
 (segment (start 138 81.77868) (end 138 71.92132) (width 0.7) (layer "F.Cu") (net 11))
 (segment (start 105.36066 63.76066) (end 100.53934 58.93934) (width 0.7) (layer "F.Cu") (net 11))
 (via (at 119.5 92.8) (size 0.7) (drill 0.5) (layers "F.Cu" "B.Cu") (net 11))
 (arc (start 137.56066 82.83934) (mid 137.885819 82.352705) (end 138 81.77868) (width 0.7) (layer "F.Cu") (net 11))
 (arc (start 131.33934 64.63934) (mid 130.852705 64.314181) (end 130.27868 64.2) (width 0.7) (layer "F.Cu") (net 11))
 (arc (start 126.97868 92.8) (mid 127.552705 92.685819) (end 128.03934 92.36066) (width 0.7) (layer "F.Cu") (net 11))
 (arc (start 100.53934 58.93934) (mid 100.214181 58.452705) (end 100.1 57.87868) (width 0.7) (layer "F.Cu") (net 11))
 (arc (start 138 71.92132) (mid 137.885819 71.347295) (end 137.56066 70.86066) (width 0.7) (layer "F.Cu") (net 11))
 (arc (start 106.42132 64.2) (mid 105.847295 64.085819) (end 105.36066 63.76066) (width 0.7) (layer "F.Cu") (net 11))
 (segment (start 119.5 92.8) (end 102.6 92.8) (width 0.7) (layer "B.Cu") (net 11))
 (segment (start 94.1 60.07868) (end 94.1 38.8) (width 0.7) (layer "F.Cu") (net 5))
 (segment (start 132.96066 72.46066) (end 129.83934 69.33934) (width 0.7) (layer "F.Cu") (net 5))
 (segment (start 133.4 80.37868) (end 133.4 73.52132) (width 0.7) (layer "F.Cu") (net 5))
 (segment (start 128.03934 86.36066) (end 132.96066 81.43934) (width 0.7) (layer "F.Cu") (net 5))
 (segment (start 122.2 86.8) (end 126.97868 86.8) (width 0.7) (layer "F.Cu") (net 5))
 (segment (start 101.86066 68.46066) (end 94.53934 61.13934) (width 0.7) (layer "F.Cu") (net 5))
 (segment (start 128.77868 68.9) (end 102.92132 68.9) (width 0.7) (layer "F.Cu") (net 5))
 (via (at 122.2 86.8) (size 0.7) (drill 0.5) (layers "F.Cu" "B.Cu") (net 5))
 (arc (start 126.97868 86.8) (mid 127.552705 86.685819) (end 128.03934 86.36066) (width 0.7) (layer "F.Cu") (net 5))
 (arc (start 102.92132 68.9) (mid 102.347295 68.785819) (end 101.86066 68.46066) (width 0.7) (layer "F.Cu") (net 5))
 (arc (start 132.96066 81.43934) (mid 133.285819 80.952705) (end 133.4 80.37868) (width 0.7) (layer "F.Cu") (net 5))
 (arc (start 94.53934 61.13934) (mid 94.214181 60.652705) (end 94.1 60.07868) (width 0.7) (layer "F.Cu") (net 5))
 (arc (start 133.4 73.52132) (mid 133.285819 72.947295) (end 132.96066 72.46066) (width 0.7) (layer "F.Cu") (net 5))
 (arc (start 129.83934 69.33934) (mid 129.352705 69.014181) (end 128.77868 68.9) (width 0.7) (layer "F.Cu") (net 5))
 (segment (start 122.2 86.8) (end 102.6 86.8) (width 0.7) (layer "B.Cu") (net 5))
 (segment (start 131.56066 73.46066) (end 128.83934 70.73934) (width 0.7) (layer "F.Cu") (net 3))
 (segment (start 127.77868 70.3) (end 101.52132 70.3) (width 0.7) (layer "F.Cu") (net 3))
 (segment (start 132 79.77868) (end 132 74.52132) (width 0.7) (layer "F.Cu") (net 3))
 (segment (start 128.03934 84.36066) (end 131.56066 80.83934) (width 0.7) (layer "F.Cu") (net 3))
 (segment (start 119.5 84.8) (end 126.97868 84.8) (width 0.7) (layer "F.Cu") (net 3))
 (segment (start 100.46066 69.86066) (end 92.53934 61.93934) (width 0.7) (layer "F.Cu") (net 3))
 (segment (start 92.1 60.87868) (end 92.1 38.8) (width 0.7) (layer "F.Cu") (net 3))
 (via (at 119.5 84.8) (size 0.7) (drill 0.5) (layers "F.Cu" "B.Cu") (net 3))
 (arc (start 126.97868 84.8) (mid 127.552705 84.685819) (end 128.03934 84.36066) (width 0.7) (layer "F.Cu") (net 3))
 (arc (start 92.53934 61.93934) (mid 92.214181 61.452705) (end 92.1 60.87868) (width 0.7) (layer "F.Cu") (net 3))
 (arc (start 101.52132 70.3) (mid 100.947295 70.185819) (end 100.46066 69.86066) (width 0.7) (layer "F.Cu") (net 3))
 (arc (start 128.83934 70.73934) (mid 128.352705 70.414181) (end 127.77868 70.3) (width 0.7) (layer "F.Cu") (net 3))
 (arc (start 132 74.52132) (mid 131.885819 73.947295) (end 131.56066 73.46066) (width 0.7) (layer "F.Cu") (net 3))
 (arc (start 131.56066 80.83934) (mid 131.885819 80.352705) (end 132 79.77868) (width 0.7) (layer "F.Cu") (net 3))
 (segment (start 119.5 84.8) (end 102.6 84.8) (width 0.7) (layer "B.Cu") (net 3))
 (segment (start 130.6 79.47868) (end 130.6 75.12132) (width 0.7) (layer "F.Cu") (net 1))
 (segment (start 128.33934 82.36066) (end 130.16066 80.53934) (width 0.7) (layer "F.Cu") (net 1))
 (segment (start 122.2 82.8) (end 127.27868 82.8) (width 0.7) (layer "F.Cu") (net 1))
 (segment (start 99.46066 71.46066) (end 90.53934 62.53934) (width 0.7) (layer "F.Cu") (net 1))
 (segment (start 127.37868 71.9) (end 100.52132 71.9) (width 0.7) (layer "F.Cu") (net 1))
 (segment (start 130.16066 74.06066) (end 128.43934 72.33934) (width 0.7) (layer "F.Cu") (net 1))
 (segment (start 90.1 61.47868) (end 90.1 38.8) (width 0.7) (layer "F.Cu") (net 1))
 (via (at 122.2 82.8) (size 0.7) (drill 0.5) (layers "F.Cu" "B.Cu") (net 1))
 (arc (start 128.43934 72.33934) (mid 127.952705 72.014181) (end 127.37868 71.9) (width 0.7) (layer "F.Cu") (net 1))
 (arc (start 130.6 75.12132) (mid 130.485819 74.547295) (end 130.16066 74.06066) (width 0.7) (layer "F.Cu") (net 1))
 (arc (start 90.53934 62.53934) (mid 90.214181 62.052705) (end 90.1 61.47868) (width 0.7) (layer "F.Cu") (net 1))
 (arc (start 100.52132 71.9) (mid 99.947295 71.785819) (end 99.46066 71.46066) (width 0.7) (layer "F.Cu") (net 1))
 (arc (start 127.27868 82.8) (mid 127.852705 82.685819) (end 128.33934 82.36066) (width 0.7) (layer "F.Cu") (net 1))
 (arc (start 130.16066 80.53934) (mid 130.485819 80.052705) (end 130.6 79.47868) (width 0.7) (layer "F.Cu") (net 1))
 (segment (start 122.2 82.8) (end 102.6 82.8) (width 0.7) (layer "B.Cu") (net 1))
 (segment (start 122.2 94.8) (end 127.07868 94.8) (width 0.7) (layer "F.Cu") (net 13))
 (segment (start 138.96066 70.76066) (end 131.53934 63.33934) (width 0.7) (layer "F.Cu") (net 13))
 (segment (start 128.13934 94.36066) (end 138.96066 83.53934) (width 0.7) (layer "F.Cu") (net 13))
 (segment (start 130.47868 62.9) (end 107.72132 62.9) (width 0.7) (layer "F.Cu") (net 13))
 (segment (start 139.4 82.47868) (end 139.4 71.82132) (width 0.7) (layer "F.Cu") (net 13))
 (segment (start 106.66066 62.46066) (end 102.53934 58.33934) (width 0.7) (layer "F.Cu") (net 13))
 (segment (start 102.1 57.27868) (end 102.1 38.8) (width 0.7) (layer "F.Cu") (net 13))
 (via (at 122.2 94.8) (size 0.7) (drill 0.5) (layers "F.Cu" "B.Cu") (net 13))
 (arc (start 131.53934 63.33934) (mid 131.052705 63.014181) (end 130.47868 62.9) (width 0.7) (layer "F.Cu") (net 13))
 (arc (start 127.07868 94.8) (mid 127.652705 94.685819) (end 128.13934 94.36066) (width 0.7) (layer "F.Cu") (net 13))
 (arc (start 102.53934 58.33934) (mid 102.214181 57.852705) (end 102.1 57.27868) (width 0.7) (layer "F.Cu") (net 13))
 (arc (start 138.96066 83.53934) (mid 139.285819 83.052705) (end 139.4 82.47868) (width 0.7) (layer "F.Cu") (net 13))
 (arc (start 107.72132 62.9) (mid 107.147295 62.785819) (end 106.66066 62.46066) (width 0.7) (layer "F.Cu") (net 13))
 (arc (start 139.4 71.82132) (mid 139.285819 71.247295) (end 138.96066 70.76066) (width 0.7) (layer "F.Cu") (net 13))
 (segment (start 122.2 94.8) (end 102.6 94.8) (width 0.7) (layer "B.Cu") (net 13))
 (segment (start 108.27266 61.15566) (end 104.53934 57.42234) (width 0.7) (layer "F.Cu") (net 15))
 (segment (start 130.82368 61.595) (end 109.33332 61.595) (width 0.7) (layer "F.Cu") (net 15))
 (segment (start 119.5 96.8) (end 127.17868 96.8) (width 0.7) (layer "F.Cu") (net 15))
 (segment (start 140.716 83.26268) (end 140.716 71.48732) (width 0.7) (layer "F.Cu") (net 15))
 (segment (start 104.1 56.36168) (end 104.1 38.8) (width 0.7) (layer "F.Cu") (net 15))
 (segment (start 128.23934 96.36066) (end 140.27666 84.32334) (width 0.7) (layer "F.Cu") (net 15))
 (segment (start 140.27666 70.42666) (end 131.88434 62.03434) (width 0.7) (layer "F.Cu") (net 15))
 (via (at 119.5 96.8) (size 0.7) (drill 0.5) (layers "F.Cu" "B.Cu") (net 15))
 (arc (start 140.27666 84.32334) (mid 140.601819 83.836705) (end 140.716 83.26268) (width 0.7) (layer "F.Cu") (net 15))
 (arc (start 104.53934 57.42234) (mid 104.214181 56.935705) (end 104.1 56.36168) (width 0.7) (layer "F.Cu") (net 15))
 (arc (start 140.716 71.48732) (mid 140.601819 70.913295) (end 140.27666 70.42666) (width 0.7) (layer "F.Cu") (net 15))
 (arc (start 109.33332 61.595) (mid 108.759295 61.480819) (end 108.27266 61.15566) (width 0.7) (layer "F.Cu") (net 15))
 (arc (start 131.88434 62.03434) (mid 131.397705 61.709181) (end 130.82368 61.595) (width 0.7) (layer "F.Cu") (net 15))
 (arc (start 127.17868 96.8) (mid 127.752705 96.685819) (end 128.23934 96.36066) (width 0.7) (layer "F.Cu") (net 15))
 (segment (start 119.5 96.8) (end 102.6 96.8) (width 0.7) (layer "B.Cu") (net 15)))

